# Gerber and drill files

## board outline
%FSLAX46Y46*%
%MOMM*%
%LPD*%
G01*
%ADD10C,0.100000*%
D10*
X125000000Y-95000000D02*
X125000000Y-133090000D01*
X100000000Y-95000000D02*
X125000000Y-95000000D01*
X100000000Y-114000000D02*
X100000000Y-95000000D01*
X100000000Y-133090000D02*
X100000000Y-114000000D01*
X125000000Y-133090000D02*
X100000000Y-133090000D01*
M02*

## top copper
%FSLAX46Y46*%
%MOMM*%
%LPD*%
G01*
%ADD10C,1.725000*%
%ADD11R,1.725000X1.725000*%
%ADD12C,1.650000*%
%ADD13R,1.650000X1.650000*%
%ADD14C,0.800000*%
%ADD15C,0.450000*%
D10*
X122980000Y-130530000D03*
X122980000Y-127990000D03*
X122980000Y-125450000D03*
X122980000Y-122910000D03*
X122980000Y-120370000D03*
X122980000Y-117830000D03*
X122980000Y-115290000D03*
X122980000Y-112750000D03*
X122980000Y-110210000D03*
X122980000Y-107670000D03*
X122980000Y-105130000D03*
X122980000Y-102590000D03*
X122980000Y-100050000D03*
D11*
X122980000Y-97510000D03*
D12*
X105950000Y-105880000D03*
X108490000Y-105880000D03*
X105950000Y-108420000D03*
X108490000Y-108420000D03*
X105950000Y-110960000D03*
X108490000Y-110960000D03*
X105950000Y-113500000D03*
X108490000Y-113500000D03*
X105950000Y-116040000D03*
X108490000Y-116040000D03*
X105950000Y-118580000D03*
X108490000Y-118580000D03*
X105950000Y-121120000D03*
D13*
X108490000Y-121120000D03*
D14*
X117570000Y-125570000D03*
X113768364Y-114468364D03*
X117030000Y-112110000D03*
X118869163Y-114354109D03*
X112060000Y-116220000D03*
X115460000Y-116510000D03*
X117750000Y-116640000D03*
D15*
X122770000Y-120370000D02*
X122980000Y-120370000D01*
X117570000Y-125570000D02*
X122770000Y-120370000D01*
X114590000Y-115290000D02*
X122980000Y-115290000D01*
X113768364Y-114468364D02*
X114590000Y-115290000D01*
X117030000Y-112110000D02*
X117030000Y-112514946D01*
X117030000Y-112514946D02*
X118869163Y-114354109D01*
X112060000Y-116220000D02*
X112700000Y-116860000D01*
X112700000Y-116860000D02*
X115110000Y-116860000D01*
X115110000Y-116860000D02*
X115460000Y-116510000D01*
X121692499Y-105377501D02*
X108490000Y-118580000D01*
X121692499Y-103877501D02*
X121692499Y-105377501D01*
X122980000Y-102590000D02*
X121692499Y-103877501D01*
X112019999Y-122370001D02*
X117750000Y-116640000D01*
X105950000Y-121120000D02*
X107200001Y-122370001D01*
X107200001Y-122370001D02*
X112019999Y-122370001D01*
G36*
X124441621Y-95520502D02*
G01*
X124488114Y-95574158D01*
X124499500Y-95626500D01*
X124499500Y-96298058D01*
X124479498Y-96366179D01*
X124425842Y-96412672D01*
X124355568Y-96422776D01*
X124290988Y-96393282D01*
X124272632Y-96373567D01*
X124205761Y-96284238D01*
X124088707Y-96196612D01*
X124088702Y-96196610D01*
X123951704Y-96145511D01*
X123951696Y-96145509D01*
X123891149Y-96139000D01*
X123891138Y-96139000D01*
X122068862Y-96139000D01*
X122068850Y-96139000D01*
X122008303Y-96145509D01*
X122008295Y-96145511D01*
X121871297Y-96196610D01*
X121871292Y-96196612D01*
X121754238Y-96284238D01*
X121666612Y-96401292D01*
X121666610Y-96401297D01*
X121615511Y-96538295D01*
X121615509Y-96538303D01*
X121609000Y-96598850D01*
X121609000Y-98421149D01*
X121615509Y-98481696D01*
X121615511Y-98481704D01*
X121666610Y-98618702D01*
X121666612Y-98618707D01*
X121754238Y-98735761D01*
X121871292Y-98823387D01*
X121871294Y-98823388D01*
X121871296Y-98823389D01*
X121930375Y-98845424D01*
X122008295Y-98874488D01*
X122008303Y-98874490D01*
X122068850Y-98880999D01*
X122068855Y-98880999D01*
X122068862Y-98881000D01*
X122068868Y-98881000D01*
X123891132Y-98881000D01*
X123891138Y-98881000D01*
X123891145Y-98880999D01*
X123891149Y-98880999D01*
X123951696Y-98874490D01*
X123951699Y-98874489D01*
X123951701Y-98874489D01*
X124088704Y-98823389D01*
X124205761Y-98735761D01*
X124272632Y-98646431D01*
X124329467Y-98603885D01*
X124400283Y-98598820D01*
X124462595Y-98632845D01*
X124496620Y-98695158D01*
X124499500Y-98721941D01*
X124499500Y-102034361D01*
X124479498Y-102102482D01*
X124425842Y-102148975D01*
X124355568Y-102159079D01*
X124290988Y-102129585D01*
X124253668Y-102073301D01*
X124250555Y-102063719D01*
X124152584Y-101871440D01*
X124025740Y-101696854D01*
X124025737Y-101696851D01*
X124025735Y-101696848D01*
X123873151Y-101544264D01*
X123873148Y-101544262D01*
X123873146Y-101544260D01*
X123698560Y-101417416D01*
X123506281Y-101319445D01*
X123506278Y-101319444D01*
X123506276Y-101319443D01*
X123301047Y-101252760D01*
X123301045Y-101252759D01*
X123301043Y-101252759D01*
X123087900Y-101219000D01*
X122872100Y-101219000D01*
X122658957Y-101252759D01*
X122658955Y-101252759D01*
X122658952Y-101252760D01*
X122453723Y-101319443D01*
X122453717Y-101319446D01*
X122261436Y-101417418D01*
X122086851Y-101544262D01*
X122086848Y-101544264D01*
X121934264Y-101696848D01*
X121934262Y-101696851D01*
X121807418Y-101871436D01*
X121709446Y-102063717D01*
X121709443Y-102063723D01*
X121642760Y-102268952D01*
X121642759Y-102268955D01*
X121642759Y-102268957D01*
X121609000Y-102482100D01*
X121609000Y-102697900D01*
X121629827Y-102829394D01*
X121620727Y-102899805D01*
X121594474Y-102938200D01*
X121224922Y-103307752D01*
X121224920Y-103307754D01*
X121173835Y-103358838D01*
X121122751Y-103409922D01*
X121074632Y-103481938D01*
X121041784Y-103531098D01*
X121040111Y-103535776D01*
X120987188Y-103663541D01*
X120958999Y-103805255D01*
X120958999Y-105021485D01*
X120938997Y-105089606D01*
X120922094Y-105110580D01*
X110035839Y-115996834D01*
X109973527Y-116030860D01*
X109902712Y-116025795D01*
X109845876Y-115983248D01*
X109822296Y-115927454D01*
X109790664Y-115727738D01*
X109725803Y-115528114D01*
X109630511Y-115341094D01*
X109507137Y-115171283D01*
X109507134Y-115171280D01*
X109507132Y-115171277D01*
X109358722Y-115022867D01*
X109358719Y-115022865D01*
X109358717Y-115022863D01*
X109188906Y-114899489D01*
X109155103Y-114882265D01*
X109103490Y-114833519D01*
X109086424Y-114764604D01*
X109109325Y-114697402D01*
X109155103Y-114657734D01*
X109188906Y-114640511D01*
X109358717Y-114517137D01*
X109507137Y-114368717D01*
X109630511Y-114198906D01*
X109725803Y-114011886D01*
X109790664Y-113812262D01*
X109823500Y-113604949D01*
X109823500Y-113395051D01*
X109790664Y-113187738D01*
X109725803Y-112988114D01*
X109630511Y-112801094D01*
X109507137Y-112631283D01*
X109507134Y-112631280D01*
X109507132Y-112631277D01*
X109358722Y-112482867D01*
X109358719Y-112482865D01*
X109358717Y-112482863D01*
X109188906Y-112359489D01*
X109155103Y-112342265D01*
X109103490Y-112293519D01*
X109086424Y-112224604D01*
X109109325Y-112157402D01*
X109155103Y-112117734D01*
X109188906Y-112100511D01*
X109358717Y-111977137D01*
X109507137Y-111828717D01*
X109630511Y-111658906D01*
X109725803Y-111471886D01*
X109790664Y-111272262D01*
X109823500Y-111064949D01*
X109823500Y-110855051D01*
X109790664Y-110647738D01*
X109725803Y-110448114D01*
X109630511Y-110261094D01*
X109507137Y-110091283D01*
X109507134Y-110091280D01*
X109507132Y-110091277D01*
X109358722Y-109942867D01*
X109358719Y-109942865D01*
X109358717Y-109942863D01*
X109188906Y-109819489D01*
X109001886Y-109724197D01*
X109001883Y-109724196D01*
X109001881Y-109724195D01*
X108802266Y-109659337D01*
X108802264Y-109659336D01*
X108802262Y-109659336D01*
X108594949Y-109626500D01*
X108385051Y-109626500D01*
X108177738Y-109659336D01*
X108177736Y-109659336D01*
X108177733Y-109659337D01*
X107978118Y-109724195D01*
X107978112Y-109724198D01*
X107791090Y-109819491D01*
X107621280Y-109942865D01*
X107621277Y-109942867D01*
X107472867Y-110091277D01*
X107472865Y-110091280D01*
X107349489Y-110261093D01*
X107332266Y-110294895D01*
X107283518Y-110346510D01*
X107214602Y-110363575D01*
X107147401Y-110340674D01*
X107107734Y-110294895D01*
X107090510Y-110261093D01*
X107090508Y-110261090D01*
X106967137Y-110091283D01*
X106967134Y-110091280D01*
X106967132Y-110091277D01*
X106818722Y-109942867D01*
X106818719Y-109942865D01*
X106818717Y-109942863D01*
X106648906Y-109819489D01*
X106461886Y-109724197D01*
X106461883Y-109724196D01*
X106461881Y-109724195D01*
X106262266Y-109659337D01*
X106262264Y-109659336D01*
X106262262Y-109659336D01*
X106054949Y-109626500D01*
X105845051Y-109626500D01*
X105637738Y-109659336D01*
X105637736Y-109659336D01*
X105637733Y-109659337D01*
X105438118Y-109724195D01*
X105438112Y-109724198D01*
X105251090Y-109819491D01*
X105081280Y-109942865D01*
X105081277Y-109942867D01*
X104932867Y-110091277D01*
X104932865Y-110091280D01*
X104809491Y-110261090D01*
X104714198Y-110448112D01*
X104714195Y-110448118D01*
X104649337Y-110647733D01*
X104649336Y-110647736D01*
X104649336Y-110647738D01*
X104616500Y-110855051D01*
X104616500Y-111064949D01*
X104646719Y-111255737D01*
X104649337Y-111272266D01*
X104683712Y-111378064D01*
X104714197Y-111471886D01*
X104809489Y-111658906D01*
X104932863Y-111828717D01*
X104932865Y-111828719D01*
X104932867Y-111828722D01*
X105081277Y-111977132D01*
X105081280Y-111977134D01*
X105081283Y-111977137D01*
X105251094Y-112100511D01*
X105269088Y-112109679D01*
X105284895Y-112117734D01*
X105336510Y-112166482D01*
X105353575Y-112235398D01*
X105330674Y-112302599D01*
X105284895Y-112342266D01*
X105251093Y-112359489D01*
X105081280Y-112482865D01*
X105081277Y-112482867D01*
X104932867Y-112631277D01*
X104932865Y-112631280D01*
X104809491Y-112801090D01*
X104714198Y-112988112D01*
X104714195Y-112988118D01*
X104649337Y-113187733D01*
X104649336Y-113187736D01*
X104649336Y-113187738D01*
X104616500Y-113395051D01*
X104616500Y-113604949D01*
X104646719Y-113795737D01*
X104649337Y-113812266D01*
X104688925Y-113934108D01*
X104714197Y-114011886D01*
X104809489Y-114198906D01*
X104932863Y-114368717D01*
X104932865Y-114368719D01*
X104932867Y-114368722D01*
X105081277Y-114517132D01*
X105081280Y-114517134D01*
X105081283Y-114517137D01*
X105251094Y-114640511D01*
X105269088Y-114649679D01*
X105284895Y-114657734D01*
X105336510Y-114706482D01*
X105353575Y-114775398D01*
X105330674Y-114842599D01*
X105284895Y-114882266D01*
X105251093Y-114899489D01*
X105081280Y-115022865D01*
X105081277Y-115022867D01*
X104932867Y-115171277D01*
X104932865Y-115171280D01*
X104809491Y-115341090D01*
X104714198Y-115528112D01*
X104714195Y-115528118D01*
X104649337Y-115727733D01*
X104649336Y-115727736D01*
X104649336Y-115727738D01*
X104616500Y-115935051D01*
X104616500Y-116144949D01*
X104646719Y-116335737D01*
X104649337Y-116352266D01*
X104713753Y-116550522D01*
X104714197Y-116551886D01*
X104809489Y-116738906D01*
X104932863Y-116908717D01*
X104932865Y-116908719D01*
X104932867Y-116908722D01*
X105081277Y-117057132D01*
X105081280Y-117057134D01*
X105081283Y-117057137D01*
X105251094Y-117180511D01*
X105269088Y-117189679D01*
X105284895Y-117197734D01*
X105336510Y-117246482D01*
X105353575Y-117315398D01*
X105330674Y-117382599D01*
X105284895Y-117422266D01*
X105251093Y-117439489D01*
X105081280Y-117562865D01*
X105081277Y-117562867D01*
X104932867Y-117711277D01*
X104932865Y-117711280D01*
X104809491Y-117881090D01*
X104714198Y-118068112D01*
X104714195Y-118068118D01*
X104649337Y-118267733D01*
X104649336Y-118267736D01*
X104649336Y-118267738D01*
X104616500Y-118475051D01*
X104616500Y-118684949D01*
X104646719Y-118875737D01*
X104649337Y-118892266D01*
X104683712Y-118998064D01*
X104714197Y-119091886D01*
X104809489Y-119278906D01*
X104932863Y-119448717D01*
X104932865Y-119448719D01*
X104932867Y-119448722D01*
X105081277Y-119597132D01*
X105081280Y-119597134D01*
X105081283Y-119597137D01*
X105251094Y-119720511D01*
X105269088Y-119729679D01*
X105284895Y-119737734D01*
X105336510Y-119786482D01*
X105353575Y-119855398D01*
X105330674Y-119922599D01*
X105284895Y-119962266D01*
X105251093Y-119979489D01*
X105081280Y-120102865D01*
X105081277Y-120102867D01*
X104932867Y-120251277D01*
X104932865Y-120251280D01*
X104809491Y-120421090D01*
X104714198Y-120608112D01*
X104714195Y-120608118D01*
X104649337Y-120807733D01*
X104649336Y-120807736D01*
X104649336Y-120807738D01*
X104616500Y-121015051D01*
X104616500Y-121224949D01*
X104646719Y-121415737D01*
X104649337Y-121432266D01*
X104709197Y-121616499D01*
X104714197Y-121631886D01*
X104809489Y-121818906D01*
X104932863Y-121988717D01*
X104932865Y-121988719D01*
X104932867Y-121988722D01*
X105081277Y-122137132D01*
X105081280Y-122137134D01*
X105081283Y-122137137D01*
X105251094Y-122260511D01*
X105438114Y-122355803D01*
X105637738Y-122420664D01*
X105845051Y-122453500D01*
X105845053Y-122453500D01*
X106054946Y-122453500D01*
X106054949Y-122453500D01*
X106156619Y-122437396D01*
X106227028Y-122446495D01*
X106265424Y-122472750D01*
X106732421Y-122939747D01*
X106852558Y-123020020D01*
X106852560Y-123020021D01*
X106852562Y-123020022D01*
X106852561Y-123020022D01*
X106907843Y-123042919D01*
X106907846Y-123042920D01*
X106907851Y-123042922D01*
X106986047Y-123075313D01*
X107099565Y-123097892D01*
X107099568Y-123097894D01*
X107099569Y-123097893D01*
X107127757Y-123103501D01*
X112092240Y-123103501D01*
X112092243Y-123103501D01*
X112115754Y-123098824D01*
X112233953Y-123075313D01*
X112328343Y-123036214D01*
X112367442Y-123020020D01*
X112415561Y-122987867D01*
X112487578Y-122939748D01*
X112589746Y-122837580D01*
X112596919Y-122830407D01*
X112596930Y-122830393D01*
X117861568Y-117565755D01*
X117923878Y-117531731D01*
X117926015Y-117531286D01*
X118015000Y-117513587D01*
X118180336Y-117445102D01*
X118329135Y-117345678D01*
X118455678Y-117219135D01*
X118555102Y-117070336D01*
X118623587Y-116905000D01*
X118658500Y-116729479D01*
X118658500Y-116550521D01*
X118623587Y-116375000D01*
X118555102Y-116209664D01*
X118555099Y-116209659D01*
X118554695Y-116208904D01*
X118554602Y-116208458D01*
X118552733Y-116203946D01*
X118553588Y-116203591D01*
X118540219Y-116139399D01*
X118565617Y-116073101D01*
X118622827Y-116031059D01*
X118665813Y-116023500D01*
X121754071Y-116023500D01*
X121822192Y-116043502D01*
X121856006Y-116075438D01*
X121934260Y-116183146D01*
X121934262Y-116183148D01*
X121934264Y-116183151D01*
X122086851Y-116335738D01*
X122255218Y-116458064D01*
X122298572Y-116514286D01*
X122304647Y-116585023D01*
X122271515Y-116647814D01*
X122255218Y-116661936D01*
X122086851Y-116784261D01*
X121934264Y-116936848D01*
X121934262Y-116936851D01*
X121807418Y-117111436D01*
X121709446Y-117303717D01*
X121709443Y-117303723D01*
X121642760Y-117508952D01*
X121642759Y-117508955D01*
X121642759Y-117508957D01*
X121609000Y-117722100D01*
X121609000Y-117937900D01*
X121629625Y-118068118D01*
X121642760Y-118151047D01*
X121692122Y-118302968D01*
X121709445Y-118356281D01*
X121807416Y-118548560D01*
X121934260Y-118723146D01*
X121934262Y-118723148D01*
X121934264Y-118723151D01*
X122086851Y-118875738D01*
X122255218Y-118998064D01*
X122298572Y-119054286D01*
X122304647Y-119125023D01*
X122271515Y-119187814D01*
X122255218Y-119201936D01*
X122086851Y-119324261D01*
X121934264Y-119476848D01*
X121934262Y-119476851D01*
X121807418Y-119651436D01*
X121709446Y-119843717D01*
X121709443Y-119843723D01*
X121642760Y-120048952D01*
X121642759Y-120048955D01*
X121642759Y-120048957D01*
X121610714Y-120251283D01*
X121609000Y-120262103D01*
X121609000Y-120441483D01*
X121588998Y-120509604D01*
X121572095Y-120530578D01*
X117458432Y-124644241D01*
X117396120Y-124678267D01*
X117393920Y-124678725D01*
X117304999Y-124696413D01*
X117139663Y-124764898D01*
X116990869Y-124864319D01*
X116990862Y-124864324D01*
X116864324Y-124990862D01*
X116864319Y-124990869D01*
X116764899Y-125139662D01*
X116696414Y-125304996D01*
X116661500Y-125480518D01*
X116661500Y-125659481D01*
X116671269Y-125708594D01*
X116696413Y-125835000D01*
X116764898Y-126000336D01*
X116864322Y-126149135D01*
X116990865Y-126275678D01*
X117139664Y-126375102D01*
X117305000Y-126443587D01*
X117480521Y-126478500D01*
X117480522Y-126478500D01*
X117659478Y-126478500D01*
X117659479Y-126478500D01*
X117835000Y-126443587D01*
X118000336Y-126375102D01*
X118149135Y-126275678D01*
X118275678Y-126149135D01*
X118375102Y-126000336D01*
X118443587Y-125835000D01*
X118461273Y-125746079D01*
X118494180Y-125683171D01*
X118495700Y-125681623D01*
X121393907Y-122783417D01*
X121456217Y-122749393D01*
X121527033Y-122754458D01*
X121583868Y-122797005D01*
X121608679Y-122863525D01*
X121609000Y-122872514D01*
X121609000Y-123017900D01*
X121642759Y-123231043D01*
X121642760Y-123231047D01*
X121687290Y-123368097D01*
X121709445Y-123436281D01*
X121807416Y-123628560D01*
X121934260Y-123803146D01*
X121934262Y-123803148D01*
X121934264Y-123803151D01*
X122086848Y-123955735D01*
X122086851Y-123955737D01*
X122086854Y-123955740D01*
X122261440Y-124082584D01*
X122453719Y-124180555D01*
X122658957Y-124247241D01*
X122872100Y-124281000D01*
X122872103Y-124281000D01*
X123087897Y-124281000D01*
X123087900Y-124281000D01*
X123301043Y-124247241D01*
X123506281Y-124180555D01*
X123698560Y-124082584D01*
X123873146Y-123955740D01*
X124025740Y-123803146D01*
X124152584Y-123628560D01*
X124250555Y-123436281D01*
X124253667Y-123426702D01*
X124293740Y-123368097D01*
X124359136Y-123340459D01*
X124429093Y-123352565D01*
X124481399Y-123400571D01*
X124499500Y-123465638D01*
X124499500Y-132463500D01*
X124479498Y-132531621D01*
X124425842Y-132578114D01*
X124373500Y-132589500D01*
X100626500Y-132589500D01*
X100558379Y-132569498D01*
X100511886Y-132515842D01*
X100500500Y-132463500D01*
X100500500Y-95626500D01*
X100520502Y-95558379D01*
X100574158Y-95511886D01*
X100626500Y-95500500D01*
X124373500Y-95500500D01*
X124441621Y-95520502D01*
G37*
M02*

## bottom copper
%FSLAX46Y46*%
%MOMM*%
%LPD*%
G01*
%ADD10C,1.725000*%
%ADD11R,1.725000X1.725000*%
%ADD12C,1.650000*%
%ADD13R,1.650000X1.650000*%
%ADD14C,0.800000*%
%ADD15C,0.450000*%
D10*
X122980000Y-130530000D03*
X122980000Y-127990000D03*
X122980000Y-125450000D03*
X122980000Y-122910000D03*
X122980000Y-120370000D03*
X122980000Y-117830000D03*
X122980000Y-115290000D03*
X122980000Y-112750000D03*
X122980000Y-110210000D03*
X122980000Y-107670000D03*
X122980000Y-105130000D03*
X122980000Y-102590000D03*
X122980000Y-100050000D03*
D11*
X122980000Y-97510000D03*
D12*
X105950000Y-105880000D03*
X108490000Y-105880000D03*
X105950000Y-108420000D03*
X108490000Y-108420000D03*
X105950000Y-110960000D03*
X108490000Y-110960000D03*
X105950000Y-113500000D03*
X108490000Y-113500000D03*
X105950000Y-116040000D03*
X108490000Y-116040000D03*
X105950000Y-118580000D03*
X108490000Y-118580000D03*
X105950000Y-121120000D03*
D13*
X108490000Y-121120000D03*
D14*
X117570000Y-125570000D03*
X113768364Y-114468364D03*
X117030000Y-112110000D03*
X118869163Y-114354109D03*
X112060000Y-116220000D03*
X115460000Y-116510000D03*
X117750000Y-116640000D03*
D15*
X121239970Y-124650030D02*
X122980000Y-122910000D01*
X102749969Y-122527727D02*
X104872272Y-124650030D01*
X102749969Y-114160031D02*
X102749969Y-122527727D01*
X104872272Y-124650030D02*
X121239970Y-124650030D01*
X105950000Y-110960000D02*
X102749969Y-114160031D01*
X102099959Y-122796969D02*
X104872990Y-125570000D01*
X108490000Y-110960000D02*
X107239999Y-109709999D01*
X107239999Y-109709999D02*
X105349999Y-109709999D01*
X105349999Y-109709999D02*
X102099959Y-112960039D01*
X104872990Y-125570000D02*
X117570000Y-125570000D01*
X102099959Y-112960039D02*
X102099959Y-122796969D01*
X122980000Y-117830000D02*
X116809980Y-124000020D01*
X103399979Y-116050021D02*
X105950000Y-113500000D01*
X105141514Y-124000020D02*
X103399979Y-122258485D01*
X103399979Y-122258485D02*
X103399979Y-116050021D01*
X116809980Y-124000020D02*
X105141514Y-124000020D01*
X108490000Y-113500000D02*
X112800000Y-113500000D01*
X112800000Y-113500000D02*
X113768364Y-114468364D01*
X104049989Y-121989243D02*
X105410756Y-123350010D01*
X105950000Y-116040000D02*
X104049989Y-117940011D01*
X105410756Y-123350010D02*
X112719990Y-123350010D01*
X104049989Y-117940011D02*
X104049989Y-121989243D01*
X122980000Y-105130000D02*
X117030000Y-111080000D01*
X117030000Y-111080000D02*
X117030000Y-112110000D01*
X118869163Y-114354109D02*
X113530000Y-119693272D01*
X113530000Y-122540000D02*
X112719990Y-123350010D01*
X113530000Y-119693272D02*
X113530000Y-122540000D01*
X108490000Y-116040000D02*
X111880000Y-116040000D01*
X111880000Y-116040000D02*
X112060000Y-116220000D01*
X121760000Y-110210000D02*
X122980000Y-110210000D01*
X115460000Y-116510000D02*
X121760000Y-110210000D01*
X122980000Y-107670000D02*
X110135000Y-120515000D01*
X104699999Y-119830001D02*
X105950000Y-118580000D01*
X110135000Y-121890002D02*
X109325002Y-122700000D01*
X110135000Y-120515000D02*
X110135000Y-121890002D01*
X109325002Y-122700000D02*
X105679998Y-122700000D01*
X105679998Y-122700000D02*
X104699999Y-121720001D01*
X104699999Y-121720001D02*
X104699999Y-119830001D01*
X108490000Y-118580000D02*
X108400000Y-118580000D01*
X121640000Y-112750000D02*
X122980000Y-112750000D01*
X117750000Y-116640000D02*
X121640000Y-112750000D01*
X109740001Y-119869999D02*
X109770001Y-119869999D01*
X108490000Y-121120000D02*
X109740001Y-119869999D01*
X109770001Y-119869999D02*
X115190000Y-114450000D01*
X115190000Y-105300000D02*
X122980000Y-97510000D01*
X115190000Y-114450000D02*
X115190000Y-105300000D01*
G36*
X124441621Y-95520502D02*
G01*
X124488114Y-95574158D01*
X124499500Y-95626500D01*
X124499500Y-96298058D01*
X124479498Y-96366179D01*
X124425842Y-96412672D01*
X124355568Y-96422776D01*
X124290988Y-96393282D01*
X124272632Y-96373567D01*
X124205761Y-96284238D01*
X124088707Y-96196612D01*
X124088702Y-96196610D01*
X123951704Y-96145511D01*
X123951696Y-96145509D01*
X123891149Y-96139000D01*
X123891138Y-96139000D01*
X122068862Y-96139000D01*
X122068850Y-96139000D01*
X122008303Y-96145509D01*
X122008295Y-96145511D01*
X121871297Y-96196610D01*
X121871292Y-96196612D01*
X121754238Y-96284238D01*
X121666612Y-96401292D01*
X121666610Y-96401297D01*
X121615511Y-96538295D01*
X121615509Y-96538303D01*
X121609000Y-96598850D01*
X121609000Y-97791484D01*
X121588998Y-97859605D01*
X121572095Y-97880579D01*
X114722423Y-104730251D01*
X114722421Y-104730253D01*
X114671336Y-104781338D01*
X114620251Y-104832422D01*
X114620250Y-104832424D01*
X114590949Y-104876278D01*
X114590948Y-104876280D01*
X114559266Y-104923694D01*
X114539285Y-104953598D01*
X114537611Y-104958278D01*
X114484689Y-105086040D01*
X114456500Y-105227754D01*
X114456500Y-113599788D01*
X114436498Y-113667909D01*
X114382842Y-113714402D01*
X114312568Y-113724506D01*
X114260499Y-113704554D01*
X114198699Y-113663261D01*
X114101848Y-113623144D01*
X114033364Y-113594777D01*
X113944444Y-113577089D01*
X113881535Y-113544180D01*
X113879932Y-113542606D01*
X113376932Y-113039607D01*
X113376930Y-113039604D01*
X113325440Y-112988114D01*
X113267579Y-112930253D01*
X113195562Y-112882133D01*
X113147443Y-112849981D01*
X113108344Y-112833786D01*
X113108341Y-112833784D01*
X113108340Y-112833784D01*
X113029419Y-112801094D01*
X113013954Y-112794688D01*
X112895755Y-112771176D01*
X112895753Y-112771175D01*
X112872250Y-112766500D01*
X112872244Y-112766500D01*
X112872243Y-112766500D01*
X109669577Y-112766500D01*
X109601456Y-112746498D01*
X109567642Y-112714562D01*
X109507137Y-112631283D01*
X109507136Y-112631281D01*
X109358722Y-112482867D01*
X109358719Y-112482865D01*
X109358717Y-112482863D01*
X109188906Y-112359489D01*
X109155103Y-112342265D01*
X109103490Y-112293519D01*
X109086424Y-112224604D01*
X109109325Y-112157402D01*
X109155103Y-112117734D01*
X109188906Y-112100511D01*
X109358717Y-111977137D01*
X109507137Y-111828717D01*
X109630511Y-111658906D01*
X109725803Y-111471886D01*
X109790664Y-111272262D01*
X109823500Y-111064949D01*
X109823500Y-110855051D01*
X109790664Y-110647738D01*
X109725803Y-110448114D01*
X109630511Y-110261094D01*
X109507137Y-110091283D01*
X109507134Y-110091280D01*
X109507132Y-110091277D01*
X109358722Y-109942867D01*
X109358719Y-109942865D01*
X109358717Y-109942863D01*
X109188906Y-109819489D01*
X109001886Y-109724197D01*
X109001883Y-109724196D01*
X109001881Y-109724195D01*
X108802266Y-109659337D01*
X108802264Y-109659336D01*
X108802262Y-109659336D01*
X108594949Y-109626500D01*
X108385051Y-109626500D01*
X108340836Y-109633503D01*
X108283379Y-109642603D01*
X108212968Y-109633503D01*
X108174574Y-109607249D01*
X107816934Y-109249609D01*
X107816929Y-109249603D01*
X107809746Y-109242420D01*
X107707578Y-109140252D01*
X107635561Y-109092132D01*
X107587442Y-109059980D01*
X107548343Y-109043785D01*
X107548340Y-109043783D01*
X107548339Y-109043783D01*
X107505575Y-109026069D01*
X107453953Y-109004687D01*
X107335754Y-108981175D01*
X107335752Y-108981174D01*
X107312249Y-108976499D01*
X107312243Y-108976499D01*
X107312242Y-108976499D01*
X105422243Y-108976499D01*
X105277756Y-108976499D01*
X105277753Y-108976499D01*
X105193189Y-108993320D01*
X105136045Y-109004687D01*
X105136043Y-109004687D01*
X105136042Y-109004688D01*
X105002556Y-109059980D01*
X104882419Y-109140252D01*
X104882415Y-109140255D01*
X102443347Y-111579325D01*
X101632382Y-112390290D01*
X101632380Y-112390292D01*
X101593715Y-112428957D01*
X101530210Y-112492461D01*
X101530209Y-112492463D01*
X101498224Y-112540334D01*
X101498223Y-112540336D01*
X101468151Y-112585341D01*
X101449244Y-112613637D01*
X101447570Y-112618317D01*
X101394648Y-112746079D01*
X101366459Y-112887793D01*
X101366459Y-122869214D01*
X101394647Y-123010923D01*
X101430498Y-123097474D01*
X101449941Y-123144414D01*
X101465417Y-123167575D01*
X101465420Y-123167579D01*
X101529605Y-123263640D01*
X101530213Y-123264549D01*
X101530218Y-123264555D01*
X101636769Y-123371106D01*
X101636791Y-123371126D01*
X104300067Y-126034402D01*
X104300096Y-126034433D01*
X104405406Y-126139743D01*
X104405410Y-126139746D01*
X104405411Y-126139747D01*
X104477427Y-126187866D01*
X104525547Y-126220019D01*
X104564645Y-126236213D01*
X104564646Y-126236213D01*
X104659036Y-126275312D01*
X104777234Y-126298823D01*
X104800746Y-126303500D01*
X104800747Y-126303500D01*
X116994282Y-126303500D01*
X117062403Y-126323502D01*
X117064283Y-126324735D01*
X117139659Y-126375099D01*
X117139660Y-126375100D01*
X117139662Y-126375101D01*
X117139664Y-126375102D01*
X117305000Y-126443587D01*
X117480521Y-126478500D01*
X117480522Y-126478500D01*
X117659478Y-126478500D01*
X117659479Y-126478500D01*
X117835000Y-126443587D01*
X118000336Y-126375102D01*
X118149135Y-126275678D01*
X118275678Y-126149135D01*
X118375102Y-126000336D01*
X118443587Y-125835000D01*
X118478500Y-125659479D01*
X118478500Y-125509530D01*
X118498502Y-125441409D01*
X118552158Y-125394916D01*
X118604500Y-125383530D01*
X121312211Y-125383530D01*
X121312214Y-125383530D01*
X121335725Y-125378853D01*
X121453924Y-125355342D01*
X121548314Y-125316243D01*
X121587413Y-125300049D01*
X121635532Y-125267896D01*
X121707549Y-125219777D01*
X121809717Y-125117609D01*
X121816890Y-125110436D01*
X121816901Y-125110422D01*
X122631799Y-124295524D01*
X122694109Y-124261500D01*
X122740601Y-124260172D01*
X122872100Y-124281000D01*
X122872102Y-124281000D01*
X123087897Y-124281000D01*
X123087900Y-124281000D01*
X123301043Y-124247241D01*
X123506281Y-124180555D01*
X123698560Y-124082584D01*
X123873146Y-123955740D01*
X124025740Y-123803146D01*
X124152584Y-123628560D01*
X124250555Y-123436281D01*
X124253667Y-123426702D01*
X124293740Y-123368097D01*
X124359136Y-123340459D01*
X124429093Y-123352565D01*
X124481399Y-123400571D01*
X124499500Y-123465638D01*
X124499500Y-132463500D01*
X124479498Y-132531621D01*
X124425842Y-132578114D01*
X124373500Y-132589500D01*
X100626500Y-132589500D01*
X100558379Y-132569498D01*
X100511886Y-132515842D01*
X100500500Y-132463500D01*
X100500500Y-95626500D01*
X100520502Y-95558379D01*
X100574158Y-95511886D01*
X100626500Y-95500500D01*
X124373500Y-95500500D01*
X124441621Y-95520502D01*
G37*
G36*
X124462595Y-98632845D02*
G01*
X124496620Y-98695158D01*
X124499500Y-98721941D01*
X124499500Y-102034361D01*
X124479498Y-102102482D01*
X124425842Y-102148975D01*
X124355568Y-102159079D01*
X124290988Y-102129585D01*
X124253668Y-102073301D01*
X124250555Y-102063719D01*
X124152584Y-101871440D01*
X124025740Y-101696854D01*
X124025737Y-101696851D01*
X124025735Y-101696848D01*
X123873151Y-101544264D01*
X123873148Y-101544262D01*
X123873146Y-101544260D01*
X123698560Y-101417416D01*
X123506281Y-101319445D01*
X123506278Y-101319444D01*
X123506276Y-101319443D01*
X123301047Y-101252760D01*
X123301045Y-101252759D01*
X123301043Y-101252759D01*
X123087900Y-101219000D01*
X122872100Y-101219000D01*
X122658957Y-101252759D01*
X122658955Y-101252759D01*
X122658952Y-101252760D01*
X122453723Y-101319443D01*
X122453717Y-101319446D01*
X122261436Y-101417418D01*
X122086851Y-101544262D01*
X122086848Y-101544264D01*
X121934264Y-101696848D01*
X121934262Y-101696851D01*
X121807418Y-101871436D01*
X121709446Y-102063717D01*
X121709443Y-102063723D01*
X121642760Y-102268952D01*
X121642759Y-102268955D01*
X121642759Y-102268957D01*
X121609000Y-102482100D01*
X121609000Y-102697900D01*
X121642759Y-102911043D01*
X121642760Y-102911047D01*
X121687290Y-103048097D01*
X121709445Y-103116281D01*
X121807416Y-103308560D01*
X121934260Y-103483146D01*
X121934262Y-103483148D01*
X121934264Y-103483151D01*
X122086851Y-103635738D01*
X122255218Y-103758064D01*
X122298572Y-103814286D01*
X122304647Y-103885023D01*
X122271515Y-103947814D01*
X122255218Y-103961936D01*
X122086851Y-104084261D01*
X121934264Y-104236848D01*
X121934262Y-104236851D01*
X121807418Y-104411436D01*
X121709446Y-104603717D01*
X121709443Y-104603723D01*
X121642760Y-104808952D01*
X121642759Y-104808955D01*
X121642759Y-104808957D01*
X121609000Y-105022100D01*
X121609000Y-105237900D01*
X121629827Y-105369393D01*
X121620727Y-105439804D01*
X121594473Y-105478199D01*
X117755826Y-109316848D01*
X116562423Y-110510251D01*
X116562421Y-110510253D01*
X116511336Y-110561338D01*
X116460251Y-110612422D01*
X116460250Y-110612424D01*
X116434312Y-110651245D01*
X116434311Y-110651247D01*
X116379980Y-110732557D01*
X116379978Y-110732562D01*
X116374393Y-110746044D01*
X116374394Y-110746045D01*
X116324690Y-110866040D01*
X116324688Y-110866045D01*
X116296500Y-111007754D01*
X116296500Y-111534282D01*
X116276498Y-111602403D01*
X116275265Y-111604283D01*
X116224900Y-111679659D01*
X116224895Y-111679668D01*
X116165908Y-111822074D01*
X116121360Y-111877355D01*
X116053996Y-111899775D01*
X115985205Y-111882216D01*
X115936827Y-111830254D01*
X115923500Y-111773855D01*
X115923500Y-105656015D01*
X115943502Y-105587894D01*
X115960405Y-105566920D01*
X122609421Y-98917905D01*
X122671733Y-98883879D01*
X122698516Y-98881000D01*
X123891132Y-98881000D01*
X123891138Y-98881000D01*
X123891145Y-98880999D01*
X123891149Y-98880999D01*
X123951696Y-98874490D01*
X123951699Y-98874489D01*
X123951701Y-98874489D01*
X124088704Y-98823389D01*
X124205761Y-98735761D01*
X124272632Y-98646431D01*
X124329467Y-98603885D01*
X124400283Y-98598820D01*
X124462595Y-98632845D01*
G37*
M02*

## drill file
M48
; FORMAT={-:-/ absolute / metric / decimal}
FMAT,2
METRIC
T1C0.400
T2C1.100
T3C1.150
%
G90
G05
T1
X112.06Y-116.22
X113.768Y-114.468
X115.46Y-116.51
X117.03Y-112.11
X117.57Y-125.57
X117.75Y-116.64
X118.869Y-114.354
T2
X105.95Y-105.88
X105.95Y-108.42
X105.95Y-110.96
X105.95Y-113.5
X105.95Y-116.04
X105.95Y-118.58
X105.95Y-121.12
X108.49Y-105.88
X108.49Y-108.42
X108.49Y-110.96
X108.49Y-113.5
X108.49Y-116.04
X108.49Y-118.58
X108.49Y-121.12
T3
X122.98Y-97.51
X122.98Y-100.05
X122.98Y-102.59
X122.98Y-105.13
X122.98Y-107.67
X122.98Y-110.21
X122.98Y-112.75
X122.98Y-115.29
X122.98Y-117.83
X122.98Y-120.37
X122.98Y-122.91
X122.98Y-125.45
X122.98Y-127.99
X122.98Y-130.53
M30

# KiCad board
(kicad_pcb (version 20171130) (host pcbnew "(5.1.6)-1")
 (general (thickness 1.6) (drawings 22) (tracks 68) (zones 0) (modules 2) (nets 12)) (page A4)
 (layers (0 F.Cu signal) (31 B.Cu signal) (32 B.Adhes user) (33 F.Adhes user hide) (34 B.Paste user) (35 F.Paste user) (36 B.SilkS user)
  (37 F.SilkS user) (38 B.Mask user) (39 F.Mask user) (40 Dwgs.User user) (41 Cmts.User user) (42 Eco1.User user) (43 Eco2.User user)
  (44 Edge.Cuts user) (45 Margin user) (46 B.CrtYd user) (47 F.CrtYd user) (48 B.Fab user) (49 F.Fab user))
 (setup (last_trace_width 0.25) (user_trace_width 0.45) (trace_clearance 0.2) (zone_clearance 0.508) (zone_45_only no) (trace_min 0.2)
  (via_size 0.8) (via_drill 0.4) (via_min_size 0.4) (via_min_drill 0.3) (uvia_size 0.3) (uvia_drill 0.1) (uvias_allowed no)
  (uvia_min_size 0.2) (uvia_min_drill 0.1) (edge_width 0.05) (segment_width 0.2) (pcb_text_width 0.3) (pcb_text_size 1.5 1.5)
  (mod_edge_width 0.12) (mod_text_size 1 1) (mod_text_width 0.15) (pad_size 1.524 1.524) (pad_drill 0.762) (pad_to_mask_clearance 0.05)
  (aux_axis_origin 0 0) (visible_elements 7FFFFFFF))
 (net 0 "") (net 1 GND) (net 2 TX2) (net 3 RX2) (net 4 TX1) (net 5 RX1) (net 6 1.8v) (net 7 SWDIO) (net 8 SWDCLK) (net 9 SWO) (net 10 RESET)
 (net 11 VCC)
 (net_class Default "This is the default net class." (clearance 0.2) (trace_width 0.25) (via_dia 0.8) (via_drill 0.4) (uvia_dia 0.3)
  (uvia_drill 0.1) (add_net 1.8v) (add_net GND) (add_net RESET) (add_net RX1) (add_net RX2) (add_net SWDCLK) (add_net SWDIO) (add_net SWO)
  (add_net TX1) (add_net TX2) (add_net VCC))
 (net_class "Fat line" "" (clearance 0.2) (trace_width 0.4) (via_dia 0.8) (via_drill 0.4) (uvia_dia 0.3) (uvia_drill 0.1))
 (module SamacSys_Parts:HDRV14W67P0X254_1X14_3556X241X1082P (layer F.Cu) (at 122.98 97.51 270)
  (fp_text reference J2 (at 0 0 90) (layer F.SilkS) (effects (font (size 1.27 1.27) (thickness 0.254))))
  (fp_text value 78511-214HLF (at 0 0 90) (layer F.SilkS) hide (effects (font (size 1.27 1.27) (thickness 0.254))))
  (pad 14 thru_hole circle (at 33.02 0 270) (size 1.725 1.725) (drill 1.15) (layers *.Cu *.Mask) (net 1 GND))
  (pad 13 thru_hole circle (at 30.48 0 270) (size 1.725 1.725) (drill 1.15) (layers *.Cu *.Mask) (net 1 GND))
  (pad 12 thru_hole circle (at 27.94 0 270) (size 1.725 1.725) (drill 1.15) (layers *.Cu *.Mask) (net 1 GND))
  (pad 11 thru_hole circle (at 25.4 0 270) (size 1.725 1.725) (drill 1.15) (layers *.Cu *.Mask) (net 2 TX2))
  (pad 10 thru_hole circle (at 22.86 0 270) (size 1.725 1.725) (drill 1.15) (layers *.Cu *.Mask) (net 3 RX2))
  (pad 9 thru_hole circle (at 20.32 0 270) (size 1.725 1.725) (drill 1.15) (layers *.Cu *.Mask) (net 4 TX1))
  (pad 8 thru_hole circle (at 17.78 0 270) (size 1.725 1.725) (drill 1.15) (layers *.Cu *.Mask) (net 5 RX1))
  (pad 7 thru_hole circle (at 15.24 0 270) (size 1.725 1.725) (drill 1.15) (layers *.Cu *.Mask) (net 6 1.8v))
  (pad 6 thru_hole circle (at 12.7 0 270) (size 1.725 1.725) (drill 1.15) (layers *.Cu *.Mask) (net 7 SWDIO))
  (pad 5 thru_hole circle (at 10.16 0 270) (size 1.725 1.725) (drill 1.15) (layers *.Cu *.Mask) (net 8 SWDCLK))
  (pad 4 thru_hole circle (at 7.62 0 270) (size 1.725 1.725) (drill 1.15) (layers *.Cu *.Mask) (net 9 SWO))
  (pad 3 thru_hole circle (at 5.08 0 270) (size 1.725 1.725) (drill 1.15) (layers *.Cu *.Mask) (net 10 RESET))
  (pad 2 thru_hole circle (at 2.54 0 270) (size 1.725 1.725) (drill 1.15) (layers *.Cu *.Mask) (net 1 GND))
  (pad 1 thru_hole rect (at 0 0 270) (size 1.725 1.725) (drill 1.15) (layers *.Cu *.Mask) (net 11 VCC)))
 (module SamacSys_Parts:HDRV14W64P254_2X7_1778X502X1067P (layer F.Cu) (at 108.49 121.12 90)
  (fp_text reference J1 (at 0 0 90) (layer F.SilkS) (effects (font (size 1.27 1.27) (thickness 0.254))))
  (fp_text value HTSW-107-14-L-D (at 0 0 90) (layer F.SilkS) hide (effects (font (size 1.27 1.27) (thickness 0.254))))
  (pad 14 thru_hole circle (at 15.24 -2.54 90) (size 1.65 1.65) (drill 1.1) (layers *.Cu *.Mask) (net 1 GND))
  (pad 13 thru_hole circle (at 15.24 0 90) (size 1.65 1.65) (drill 1.1) (layers *.Cu *.Mask) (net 1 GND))
  (pad 12 thru_hole circle (at 12.7 -2.54 90) (size 1.65 1.65) (drill 1.1) (layers *.Cu *.Mask) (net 1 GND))
  (pad 11 thru_hole circle (at 12.7 0 90) (size 1.65 1.65) (drill 1.1) (layers *.Cu *.Mask) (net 1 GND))
  (pad 10 thru_hole circle (at 10.16 -2.54 90) (size 1.65 1.65) (drill 1.1) (layers *.Cu *.Mask) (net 2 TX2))
  (pad 9 thru_hole circle (at 10.16 0 90) (size 1.65 1.65) (drill 1.1) (layers *.Cu *.Mask) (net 3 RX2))
  (pad 8 thru_hole circle (at 7.62 -2.54 90) (size 1.65 1.65) (drill 1.1) (layers *.Cu *.Mask) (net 4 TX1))
  (pad 7 thru_hole circle (at 7.62 0 90) (size 1.65 1.65) (drill 1.1) (layers *.Cu *.Mask) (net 5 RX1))
  (pad 6 thru_hole circle (at 5.08 -2.54 90) (size 1.65 1.65) (drill 1.1) (layers *.Cu *.Mask) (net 9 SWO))
  (pad 5 thru_hole circle (at 5.08 0 90) (size 1.65 1.65) (drill 1.1) (layers *.Cu *.Mask) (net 7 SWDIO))
  (pad 4 thru_hole circle (at 2.54 -2.54 90) (size 1.65 1.65) (drill 1.1) (layers *.Cu *.Mask) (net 8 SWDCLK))
  (pad 3 thru_hole circle (at 2.54 0 90) (size 1.65 1.65) (drill 1.1) (layers *.Cu *.Mask) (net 10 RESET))
  (pad 2 thru_hole circle (at 0 -2.54 90) (size 1.65 1.65) (drill 1.1) (layers *.Cu *.Mask) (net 6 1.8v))
  (pad 1 thru_hole rect (at 0 0 90) (size 1.65 1.65) (drill 1.1) (layers *.Cu *.Mask) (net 11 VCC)))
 (gr_line (start 125 95) (end 125 133.09) (layer Edge.Cuts) (width 0.1))
 (gr_line (start 100 95) (end 125 95) (layer Edge.Cuts) (width 0.1))
 (gr_line (start 100 114) (end 100 95) (layer Edge.Cuts) (width 0.1))
 (gr_line (start 100 133.09) (end 100 114) (layer Edge.Cuts) (width 0.1))
 (gr_line (start 125 133.09) (end 100 133.09) (layer Edge.Cuts) (width 0.1))
 (segment (start 121.23997 124.65003) (end 122.98 122.91) (width 0.45) (layer B.Cu) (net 2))
 (segment (start 102.749969 122.527727) (end 104.872272 124.65003) (width 0.45) (layer B.Cu) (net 2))
 (segment (start 102.749969 114.160031) (end 102.749969 122.527727) (width 0.45) (layer B.Cu) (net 2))
 (segment (start 104.872272 124.65003) (end 121.23997 124.65003) (width 0.45) (layer B.Cu) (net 2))
 (segment (start 105.95 110.96) (end 102.749969 114.160031) (width 0.45) (layer B.Cu) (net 2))
 (via (at 117.57 125.57) (size 0.8) (drill 0.4) (layers F.Cu B.Cu) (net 3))
 (segment (start 102.099959 122.796969) (end 104.87299 125.57) (width 0.45) (layer B.Cu) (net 3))
 (segment (start 108.49 110.96) (end 107.239999 109.709999) (width 0.45) (layer B.Cu) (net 3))
 (segment (start 107.239999 109.709999) (end 105.349999 109.709999) (width 0.45) (layer B.Cu) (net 3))
 (segment (start 105.349999 109.709999) (end 102.099959 112.960039) (width 0.45) (layer B.Cu) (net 3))
 (segment (start 104.87299 125.57) (end 117.57 125.57) (width 0.45) (layer B.Cu) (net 3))
 (segment (start 102.099959 112.960039) (end 102.099959 122.796969) (width 0.45) (layer B.Cu) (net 3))
 (segment (start 122.77 120.37) (end 122.98 120.37) (width 0.45) (layer F.Cu) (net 3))
 (segment (start 117.57 125.57) (end 122.77 120.37) (width 0.45) (layer F.Cu) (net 3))
 (segment (start 122.98 117.83) (end 116.80998 124.00002) (width 0.45) (layer B.Cu) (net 4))
 (segment (start 103.399979 116.050021) (end 105.95 113.5) (width 0.45) (layer B.Cu) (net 4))
 (segment (start 105.141514 124.00002) (end 103.399979 122.258485) (width 0.45) (layer B.Cu) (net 4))
 (segment (start 103.399979 122.258485) (end 103.399979 116.050021) (width 0.45) (layer B.Cu) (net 4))
 (segment (start 116.80998 124.00002) (end 105.141514 124.00002) (width 0.45) (layer B.Cu) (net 4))
 (segment (start 108.49 113.5) (end 112.8 113.5) (width 0.45) (layer B.Cu) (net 5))
 (via (at 113.768364 114.468364) (size 0.8) (drill 0.4) (layers F.Cu B.Cu) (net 5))
 (segment (start 112.8 113.5) (end 113.768364 114.468364) (width 0.45) (layer B.Cu) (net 5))
 (segment (start 114.59 115.29) (end 122.98 115.29) (width 0.45) (layer F.Cu) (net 5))
 (segment (start 113.768364 114.468364) (end 114.59 115.29) (width 0.45) (layer F.Cu) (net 5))
 (segment (start 104.049989 121.989243) (end 105.410756 123.35001) (width 0.45) (layer B.Cu) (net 9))
 (segment (start 105.95 116.04) (end 104.049989 117.940011) (width 0.45) (layer B.Cu) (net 9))
 (segment (start 105.410756 123.35001) (end 112.71999 123.35001) (width 0.45) (layer B.Cu) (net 9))
 (segment (start 104.049989 117.940011) (end 104.049989 121.989243) (width 0.45) (layer B.Cu) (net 9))
 (via (at 117.03 112.11) (size 0.8) (drill 0.4) (layers F.Cu B.Cu) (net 9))
 (segment (start 122.98 105.13) (end 117.03 111.08) (width 0.45) (layer B.Cu) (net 9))
 (segment (start 117.03 111.08) (end 117.03 112.11) (width 0.45) (layer B.Cu) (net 9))
 (via (at 118.869163 114.354109) (size 0.8) (drill 0.4) (layers F.Cu B.Cu) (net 9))
 (segment (start 117.03 112.11) (end 117.03 112.514946) (width 0.45) (layer F.Cu) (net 9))
 (segment (start 117.03 112.514946) (end 118.869163 114.354109) (width 0.45) (layer F.Cu) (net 9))
 (segment (start 118.869163 114.354109) (end 113.53 119.693272) (width 0.45) (layer B.Cu) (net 9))
 (segment (start 113.53 122.54) (end 112.71999 123.35001) (width 0.45) (layer B.Cu) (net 9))
 (segment (start 113.53 119.693272) (end 113.53 122.54) (width 0.45) (layer B.Cu) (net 9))
 (segment (start 108.49 116.04) (end 111.88 116.04) (width 0.45) (layer B.Cu) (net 7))
 (via (at 112.06 116.22) (size 0.8) (drill 0.4) (layers F.Cu B.Cu) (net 7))
 (segment (start 111.88 116.04) (end 112.06 116.22) (width 0.45) (layer B.Cu) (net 7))
 (segment (start 112.06 116.22) (end 112.7 116.86) (width 0.45) (layer F.Cu) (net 7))
 (segment (start 112.7 116.86) (end 115.11 116.86) (width 0.45) (layer F.Cu) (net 7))
 (via (at 115.46 116.51) (size 0.8) (drill 0.4) (layers F.Cu B.Cu) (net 7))
 (segment (start 115.11 116.86) (end 115.46 116.51) (width 0.45) (layer F.Cu) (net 7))
 (segment (start 121.76 110.21) (end 122.98 110.21) (width 0.45) (layer B.Cu) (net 7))
 (segment (start 115.46 116.51) (end 121.76 110.21) (width 0.45) (layer B.Cu) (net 7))
 (segment (start 122.98 107.67) (end 110.135 120.515) (width 0.45) (layer B.Cu) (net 8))
 (segment (start 104.699999 119.830001) (end 105.95 118.58) (width 0.45) (layer B.Cu) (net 8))
 (segment (start 110.135 121.890002) (end 109.325002 122.7) (width 0.45) (layer B.Cu) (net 8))
 (segment (start 110.135 120.515) (end 110.135 121.890002) (width 0.45) (layer B.Cu) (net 8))
 (segment (start 109.325002 122.7) (end 105.679998 122.7) (width 0.45) (layer B.Cu) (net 8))
 (segment (start 105.679998 122.7) (end 104.699999 121.720001) (width 0.45) (layer B.Cu) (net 8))
 (segment (start 104.699999 121.720001) (end 104.699999 119.830001) (width 0.45) (layer B.Cu) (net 8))
 (segment (start 121.692499 105.377501) (end 108.49 118.58) (width 0.45) (layer F.Cu) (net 10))
 (segment (start 121.692499 103.877501) (end 121.692499 105.377501) (width 0.45) (layer F.Cu) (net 10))
 (segment (start 122.98 102.59) (end 121.692499 103.877501) (width 0.45) (layer F.Cu) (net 10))
 (segment (start 108.49 118.58) (end 108.4 118.58) (width 0.45) (layer B.Cu) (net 10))
 (segment (start 112.019999 122.370001) (end 117.75 116.64) (width 0.45) (layer F.Cu) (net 6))
 (segment (start 105.95 121.12) (end 107.200001 122.370001) (width 0.45) (layer F.Cu) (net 6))
 (via (at 117.75 116.64) (size 0.8) (drill 0.4) (layers F.Cu B.Cu) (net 6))
 (segment (start 107.200001 122.370001) (end 112.019999 122.370001) (width 0.45) (layer F.Cu) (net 6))
 (segment (start 121.64 112.75) (end 122.98 112.75) (width 0.45) (layer B.Cu) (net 6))
 (segment (start 117.75 116.64) (end 121.64 112.75) (width 0.45) (layer B.Cu) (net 6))
 (segment (start 109.740001 119.869999) (end 109.770001 119.869999) (width 0.45) (layer B.Cu) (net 11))
 (segment (start 108.49 121.12) (end 109.740001 119.869999) (width 0.45) (layer B.Cu) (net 11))
 (segment (start 109.770001 119.869999) (end 115.19 114.45) (width 0.45) (layer B.Cu) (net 11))
 (segment (start 115.19 105.3) (end 122.98 97.51) (width 0.45) (layer B.Cu) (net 11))
 (segment (start 115.19 114.45) (end 115.19 105.3) (width 0.45) (layer B.Cu) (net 11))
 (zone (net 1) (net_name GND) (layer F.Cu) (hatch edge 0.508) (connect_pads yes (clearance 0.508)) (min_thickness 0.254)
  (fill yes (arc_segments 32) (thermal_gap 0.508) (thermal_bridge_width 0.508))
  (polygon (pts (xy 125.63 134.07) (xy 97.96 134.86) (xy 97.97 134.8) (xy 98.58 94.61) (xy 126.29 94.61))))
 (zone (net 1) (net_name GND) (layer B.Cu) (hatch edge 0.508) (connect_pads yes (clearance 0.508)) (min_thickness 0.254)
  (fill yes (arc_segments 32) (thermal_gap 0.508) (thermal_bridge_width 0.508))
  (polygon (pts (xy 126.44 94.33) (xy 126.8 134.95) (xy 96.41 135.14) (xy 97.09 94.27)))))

